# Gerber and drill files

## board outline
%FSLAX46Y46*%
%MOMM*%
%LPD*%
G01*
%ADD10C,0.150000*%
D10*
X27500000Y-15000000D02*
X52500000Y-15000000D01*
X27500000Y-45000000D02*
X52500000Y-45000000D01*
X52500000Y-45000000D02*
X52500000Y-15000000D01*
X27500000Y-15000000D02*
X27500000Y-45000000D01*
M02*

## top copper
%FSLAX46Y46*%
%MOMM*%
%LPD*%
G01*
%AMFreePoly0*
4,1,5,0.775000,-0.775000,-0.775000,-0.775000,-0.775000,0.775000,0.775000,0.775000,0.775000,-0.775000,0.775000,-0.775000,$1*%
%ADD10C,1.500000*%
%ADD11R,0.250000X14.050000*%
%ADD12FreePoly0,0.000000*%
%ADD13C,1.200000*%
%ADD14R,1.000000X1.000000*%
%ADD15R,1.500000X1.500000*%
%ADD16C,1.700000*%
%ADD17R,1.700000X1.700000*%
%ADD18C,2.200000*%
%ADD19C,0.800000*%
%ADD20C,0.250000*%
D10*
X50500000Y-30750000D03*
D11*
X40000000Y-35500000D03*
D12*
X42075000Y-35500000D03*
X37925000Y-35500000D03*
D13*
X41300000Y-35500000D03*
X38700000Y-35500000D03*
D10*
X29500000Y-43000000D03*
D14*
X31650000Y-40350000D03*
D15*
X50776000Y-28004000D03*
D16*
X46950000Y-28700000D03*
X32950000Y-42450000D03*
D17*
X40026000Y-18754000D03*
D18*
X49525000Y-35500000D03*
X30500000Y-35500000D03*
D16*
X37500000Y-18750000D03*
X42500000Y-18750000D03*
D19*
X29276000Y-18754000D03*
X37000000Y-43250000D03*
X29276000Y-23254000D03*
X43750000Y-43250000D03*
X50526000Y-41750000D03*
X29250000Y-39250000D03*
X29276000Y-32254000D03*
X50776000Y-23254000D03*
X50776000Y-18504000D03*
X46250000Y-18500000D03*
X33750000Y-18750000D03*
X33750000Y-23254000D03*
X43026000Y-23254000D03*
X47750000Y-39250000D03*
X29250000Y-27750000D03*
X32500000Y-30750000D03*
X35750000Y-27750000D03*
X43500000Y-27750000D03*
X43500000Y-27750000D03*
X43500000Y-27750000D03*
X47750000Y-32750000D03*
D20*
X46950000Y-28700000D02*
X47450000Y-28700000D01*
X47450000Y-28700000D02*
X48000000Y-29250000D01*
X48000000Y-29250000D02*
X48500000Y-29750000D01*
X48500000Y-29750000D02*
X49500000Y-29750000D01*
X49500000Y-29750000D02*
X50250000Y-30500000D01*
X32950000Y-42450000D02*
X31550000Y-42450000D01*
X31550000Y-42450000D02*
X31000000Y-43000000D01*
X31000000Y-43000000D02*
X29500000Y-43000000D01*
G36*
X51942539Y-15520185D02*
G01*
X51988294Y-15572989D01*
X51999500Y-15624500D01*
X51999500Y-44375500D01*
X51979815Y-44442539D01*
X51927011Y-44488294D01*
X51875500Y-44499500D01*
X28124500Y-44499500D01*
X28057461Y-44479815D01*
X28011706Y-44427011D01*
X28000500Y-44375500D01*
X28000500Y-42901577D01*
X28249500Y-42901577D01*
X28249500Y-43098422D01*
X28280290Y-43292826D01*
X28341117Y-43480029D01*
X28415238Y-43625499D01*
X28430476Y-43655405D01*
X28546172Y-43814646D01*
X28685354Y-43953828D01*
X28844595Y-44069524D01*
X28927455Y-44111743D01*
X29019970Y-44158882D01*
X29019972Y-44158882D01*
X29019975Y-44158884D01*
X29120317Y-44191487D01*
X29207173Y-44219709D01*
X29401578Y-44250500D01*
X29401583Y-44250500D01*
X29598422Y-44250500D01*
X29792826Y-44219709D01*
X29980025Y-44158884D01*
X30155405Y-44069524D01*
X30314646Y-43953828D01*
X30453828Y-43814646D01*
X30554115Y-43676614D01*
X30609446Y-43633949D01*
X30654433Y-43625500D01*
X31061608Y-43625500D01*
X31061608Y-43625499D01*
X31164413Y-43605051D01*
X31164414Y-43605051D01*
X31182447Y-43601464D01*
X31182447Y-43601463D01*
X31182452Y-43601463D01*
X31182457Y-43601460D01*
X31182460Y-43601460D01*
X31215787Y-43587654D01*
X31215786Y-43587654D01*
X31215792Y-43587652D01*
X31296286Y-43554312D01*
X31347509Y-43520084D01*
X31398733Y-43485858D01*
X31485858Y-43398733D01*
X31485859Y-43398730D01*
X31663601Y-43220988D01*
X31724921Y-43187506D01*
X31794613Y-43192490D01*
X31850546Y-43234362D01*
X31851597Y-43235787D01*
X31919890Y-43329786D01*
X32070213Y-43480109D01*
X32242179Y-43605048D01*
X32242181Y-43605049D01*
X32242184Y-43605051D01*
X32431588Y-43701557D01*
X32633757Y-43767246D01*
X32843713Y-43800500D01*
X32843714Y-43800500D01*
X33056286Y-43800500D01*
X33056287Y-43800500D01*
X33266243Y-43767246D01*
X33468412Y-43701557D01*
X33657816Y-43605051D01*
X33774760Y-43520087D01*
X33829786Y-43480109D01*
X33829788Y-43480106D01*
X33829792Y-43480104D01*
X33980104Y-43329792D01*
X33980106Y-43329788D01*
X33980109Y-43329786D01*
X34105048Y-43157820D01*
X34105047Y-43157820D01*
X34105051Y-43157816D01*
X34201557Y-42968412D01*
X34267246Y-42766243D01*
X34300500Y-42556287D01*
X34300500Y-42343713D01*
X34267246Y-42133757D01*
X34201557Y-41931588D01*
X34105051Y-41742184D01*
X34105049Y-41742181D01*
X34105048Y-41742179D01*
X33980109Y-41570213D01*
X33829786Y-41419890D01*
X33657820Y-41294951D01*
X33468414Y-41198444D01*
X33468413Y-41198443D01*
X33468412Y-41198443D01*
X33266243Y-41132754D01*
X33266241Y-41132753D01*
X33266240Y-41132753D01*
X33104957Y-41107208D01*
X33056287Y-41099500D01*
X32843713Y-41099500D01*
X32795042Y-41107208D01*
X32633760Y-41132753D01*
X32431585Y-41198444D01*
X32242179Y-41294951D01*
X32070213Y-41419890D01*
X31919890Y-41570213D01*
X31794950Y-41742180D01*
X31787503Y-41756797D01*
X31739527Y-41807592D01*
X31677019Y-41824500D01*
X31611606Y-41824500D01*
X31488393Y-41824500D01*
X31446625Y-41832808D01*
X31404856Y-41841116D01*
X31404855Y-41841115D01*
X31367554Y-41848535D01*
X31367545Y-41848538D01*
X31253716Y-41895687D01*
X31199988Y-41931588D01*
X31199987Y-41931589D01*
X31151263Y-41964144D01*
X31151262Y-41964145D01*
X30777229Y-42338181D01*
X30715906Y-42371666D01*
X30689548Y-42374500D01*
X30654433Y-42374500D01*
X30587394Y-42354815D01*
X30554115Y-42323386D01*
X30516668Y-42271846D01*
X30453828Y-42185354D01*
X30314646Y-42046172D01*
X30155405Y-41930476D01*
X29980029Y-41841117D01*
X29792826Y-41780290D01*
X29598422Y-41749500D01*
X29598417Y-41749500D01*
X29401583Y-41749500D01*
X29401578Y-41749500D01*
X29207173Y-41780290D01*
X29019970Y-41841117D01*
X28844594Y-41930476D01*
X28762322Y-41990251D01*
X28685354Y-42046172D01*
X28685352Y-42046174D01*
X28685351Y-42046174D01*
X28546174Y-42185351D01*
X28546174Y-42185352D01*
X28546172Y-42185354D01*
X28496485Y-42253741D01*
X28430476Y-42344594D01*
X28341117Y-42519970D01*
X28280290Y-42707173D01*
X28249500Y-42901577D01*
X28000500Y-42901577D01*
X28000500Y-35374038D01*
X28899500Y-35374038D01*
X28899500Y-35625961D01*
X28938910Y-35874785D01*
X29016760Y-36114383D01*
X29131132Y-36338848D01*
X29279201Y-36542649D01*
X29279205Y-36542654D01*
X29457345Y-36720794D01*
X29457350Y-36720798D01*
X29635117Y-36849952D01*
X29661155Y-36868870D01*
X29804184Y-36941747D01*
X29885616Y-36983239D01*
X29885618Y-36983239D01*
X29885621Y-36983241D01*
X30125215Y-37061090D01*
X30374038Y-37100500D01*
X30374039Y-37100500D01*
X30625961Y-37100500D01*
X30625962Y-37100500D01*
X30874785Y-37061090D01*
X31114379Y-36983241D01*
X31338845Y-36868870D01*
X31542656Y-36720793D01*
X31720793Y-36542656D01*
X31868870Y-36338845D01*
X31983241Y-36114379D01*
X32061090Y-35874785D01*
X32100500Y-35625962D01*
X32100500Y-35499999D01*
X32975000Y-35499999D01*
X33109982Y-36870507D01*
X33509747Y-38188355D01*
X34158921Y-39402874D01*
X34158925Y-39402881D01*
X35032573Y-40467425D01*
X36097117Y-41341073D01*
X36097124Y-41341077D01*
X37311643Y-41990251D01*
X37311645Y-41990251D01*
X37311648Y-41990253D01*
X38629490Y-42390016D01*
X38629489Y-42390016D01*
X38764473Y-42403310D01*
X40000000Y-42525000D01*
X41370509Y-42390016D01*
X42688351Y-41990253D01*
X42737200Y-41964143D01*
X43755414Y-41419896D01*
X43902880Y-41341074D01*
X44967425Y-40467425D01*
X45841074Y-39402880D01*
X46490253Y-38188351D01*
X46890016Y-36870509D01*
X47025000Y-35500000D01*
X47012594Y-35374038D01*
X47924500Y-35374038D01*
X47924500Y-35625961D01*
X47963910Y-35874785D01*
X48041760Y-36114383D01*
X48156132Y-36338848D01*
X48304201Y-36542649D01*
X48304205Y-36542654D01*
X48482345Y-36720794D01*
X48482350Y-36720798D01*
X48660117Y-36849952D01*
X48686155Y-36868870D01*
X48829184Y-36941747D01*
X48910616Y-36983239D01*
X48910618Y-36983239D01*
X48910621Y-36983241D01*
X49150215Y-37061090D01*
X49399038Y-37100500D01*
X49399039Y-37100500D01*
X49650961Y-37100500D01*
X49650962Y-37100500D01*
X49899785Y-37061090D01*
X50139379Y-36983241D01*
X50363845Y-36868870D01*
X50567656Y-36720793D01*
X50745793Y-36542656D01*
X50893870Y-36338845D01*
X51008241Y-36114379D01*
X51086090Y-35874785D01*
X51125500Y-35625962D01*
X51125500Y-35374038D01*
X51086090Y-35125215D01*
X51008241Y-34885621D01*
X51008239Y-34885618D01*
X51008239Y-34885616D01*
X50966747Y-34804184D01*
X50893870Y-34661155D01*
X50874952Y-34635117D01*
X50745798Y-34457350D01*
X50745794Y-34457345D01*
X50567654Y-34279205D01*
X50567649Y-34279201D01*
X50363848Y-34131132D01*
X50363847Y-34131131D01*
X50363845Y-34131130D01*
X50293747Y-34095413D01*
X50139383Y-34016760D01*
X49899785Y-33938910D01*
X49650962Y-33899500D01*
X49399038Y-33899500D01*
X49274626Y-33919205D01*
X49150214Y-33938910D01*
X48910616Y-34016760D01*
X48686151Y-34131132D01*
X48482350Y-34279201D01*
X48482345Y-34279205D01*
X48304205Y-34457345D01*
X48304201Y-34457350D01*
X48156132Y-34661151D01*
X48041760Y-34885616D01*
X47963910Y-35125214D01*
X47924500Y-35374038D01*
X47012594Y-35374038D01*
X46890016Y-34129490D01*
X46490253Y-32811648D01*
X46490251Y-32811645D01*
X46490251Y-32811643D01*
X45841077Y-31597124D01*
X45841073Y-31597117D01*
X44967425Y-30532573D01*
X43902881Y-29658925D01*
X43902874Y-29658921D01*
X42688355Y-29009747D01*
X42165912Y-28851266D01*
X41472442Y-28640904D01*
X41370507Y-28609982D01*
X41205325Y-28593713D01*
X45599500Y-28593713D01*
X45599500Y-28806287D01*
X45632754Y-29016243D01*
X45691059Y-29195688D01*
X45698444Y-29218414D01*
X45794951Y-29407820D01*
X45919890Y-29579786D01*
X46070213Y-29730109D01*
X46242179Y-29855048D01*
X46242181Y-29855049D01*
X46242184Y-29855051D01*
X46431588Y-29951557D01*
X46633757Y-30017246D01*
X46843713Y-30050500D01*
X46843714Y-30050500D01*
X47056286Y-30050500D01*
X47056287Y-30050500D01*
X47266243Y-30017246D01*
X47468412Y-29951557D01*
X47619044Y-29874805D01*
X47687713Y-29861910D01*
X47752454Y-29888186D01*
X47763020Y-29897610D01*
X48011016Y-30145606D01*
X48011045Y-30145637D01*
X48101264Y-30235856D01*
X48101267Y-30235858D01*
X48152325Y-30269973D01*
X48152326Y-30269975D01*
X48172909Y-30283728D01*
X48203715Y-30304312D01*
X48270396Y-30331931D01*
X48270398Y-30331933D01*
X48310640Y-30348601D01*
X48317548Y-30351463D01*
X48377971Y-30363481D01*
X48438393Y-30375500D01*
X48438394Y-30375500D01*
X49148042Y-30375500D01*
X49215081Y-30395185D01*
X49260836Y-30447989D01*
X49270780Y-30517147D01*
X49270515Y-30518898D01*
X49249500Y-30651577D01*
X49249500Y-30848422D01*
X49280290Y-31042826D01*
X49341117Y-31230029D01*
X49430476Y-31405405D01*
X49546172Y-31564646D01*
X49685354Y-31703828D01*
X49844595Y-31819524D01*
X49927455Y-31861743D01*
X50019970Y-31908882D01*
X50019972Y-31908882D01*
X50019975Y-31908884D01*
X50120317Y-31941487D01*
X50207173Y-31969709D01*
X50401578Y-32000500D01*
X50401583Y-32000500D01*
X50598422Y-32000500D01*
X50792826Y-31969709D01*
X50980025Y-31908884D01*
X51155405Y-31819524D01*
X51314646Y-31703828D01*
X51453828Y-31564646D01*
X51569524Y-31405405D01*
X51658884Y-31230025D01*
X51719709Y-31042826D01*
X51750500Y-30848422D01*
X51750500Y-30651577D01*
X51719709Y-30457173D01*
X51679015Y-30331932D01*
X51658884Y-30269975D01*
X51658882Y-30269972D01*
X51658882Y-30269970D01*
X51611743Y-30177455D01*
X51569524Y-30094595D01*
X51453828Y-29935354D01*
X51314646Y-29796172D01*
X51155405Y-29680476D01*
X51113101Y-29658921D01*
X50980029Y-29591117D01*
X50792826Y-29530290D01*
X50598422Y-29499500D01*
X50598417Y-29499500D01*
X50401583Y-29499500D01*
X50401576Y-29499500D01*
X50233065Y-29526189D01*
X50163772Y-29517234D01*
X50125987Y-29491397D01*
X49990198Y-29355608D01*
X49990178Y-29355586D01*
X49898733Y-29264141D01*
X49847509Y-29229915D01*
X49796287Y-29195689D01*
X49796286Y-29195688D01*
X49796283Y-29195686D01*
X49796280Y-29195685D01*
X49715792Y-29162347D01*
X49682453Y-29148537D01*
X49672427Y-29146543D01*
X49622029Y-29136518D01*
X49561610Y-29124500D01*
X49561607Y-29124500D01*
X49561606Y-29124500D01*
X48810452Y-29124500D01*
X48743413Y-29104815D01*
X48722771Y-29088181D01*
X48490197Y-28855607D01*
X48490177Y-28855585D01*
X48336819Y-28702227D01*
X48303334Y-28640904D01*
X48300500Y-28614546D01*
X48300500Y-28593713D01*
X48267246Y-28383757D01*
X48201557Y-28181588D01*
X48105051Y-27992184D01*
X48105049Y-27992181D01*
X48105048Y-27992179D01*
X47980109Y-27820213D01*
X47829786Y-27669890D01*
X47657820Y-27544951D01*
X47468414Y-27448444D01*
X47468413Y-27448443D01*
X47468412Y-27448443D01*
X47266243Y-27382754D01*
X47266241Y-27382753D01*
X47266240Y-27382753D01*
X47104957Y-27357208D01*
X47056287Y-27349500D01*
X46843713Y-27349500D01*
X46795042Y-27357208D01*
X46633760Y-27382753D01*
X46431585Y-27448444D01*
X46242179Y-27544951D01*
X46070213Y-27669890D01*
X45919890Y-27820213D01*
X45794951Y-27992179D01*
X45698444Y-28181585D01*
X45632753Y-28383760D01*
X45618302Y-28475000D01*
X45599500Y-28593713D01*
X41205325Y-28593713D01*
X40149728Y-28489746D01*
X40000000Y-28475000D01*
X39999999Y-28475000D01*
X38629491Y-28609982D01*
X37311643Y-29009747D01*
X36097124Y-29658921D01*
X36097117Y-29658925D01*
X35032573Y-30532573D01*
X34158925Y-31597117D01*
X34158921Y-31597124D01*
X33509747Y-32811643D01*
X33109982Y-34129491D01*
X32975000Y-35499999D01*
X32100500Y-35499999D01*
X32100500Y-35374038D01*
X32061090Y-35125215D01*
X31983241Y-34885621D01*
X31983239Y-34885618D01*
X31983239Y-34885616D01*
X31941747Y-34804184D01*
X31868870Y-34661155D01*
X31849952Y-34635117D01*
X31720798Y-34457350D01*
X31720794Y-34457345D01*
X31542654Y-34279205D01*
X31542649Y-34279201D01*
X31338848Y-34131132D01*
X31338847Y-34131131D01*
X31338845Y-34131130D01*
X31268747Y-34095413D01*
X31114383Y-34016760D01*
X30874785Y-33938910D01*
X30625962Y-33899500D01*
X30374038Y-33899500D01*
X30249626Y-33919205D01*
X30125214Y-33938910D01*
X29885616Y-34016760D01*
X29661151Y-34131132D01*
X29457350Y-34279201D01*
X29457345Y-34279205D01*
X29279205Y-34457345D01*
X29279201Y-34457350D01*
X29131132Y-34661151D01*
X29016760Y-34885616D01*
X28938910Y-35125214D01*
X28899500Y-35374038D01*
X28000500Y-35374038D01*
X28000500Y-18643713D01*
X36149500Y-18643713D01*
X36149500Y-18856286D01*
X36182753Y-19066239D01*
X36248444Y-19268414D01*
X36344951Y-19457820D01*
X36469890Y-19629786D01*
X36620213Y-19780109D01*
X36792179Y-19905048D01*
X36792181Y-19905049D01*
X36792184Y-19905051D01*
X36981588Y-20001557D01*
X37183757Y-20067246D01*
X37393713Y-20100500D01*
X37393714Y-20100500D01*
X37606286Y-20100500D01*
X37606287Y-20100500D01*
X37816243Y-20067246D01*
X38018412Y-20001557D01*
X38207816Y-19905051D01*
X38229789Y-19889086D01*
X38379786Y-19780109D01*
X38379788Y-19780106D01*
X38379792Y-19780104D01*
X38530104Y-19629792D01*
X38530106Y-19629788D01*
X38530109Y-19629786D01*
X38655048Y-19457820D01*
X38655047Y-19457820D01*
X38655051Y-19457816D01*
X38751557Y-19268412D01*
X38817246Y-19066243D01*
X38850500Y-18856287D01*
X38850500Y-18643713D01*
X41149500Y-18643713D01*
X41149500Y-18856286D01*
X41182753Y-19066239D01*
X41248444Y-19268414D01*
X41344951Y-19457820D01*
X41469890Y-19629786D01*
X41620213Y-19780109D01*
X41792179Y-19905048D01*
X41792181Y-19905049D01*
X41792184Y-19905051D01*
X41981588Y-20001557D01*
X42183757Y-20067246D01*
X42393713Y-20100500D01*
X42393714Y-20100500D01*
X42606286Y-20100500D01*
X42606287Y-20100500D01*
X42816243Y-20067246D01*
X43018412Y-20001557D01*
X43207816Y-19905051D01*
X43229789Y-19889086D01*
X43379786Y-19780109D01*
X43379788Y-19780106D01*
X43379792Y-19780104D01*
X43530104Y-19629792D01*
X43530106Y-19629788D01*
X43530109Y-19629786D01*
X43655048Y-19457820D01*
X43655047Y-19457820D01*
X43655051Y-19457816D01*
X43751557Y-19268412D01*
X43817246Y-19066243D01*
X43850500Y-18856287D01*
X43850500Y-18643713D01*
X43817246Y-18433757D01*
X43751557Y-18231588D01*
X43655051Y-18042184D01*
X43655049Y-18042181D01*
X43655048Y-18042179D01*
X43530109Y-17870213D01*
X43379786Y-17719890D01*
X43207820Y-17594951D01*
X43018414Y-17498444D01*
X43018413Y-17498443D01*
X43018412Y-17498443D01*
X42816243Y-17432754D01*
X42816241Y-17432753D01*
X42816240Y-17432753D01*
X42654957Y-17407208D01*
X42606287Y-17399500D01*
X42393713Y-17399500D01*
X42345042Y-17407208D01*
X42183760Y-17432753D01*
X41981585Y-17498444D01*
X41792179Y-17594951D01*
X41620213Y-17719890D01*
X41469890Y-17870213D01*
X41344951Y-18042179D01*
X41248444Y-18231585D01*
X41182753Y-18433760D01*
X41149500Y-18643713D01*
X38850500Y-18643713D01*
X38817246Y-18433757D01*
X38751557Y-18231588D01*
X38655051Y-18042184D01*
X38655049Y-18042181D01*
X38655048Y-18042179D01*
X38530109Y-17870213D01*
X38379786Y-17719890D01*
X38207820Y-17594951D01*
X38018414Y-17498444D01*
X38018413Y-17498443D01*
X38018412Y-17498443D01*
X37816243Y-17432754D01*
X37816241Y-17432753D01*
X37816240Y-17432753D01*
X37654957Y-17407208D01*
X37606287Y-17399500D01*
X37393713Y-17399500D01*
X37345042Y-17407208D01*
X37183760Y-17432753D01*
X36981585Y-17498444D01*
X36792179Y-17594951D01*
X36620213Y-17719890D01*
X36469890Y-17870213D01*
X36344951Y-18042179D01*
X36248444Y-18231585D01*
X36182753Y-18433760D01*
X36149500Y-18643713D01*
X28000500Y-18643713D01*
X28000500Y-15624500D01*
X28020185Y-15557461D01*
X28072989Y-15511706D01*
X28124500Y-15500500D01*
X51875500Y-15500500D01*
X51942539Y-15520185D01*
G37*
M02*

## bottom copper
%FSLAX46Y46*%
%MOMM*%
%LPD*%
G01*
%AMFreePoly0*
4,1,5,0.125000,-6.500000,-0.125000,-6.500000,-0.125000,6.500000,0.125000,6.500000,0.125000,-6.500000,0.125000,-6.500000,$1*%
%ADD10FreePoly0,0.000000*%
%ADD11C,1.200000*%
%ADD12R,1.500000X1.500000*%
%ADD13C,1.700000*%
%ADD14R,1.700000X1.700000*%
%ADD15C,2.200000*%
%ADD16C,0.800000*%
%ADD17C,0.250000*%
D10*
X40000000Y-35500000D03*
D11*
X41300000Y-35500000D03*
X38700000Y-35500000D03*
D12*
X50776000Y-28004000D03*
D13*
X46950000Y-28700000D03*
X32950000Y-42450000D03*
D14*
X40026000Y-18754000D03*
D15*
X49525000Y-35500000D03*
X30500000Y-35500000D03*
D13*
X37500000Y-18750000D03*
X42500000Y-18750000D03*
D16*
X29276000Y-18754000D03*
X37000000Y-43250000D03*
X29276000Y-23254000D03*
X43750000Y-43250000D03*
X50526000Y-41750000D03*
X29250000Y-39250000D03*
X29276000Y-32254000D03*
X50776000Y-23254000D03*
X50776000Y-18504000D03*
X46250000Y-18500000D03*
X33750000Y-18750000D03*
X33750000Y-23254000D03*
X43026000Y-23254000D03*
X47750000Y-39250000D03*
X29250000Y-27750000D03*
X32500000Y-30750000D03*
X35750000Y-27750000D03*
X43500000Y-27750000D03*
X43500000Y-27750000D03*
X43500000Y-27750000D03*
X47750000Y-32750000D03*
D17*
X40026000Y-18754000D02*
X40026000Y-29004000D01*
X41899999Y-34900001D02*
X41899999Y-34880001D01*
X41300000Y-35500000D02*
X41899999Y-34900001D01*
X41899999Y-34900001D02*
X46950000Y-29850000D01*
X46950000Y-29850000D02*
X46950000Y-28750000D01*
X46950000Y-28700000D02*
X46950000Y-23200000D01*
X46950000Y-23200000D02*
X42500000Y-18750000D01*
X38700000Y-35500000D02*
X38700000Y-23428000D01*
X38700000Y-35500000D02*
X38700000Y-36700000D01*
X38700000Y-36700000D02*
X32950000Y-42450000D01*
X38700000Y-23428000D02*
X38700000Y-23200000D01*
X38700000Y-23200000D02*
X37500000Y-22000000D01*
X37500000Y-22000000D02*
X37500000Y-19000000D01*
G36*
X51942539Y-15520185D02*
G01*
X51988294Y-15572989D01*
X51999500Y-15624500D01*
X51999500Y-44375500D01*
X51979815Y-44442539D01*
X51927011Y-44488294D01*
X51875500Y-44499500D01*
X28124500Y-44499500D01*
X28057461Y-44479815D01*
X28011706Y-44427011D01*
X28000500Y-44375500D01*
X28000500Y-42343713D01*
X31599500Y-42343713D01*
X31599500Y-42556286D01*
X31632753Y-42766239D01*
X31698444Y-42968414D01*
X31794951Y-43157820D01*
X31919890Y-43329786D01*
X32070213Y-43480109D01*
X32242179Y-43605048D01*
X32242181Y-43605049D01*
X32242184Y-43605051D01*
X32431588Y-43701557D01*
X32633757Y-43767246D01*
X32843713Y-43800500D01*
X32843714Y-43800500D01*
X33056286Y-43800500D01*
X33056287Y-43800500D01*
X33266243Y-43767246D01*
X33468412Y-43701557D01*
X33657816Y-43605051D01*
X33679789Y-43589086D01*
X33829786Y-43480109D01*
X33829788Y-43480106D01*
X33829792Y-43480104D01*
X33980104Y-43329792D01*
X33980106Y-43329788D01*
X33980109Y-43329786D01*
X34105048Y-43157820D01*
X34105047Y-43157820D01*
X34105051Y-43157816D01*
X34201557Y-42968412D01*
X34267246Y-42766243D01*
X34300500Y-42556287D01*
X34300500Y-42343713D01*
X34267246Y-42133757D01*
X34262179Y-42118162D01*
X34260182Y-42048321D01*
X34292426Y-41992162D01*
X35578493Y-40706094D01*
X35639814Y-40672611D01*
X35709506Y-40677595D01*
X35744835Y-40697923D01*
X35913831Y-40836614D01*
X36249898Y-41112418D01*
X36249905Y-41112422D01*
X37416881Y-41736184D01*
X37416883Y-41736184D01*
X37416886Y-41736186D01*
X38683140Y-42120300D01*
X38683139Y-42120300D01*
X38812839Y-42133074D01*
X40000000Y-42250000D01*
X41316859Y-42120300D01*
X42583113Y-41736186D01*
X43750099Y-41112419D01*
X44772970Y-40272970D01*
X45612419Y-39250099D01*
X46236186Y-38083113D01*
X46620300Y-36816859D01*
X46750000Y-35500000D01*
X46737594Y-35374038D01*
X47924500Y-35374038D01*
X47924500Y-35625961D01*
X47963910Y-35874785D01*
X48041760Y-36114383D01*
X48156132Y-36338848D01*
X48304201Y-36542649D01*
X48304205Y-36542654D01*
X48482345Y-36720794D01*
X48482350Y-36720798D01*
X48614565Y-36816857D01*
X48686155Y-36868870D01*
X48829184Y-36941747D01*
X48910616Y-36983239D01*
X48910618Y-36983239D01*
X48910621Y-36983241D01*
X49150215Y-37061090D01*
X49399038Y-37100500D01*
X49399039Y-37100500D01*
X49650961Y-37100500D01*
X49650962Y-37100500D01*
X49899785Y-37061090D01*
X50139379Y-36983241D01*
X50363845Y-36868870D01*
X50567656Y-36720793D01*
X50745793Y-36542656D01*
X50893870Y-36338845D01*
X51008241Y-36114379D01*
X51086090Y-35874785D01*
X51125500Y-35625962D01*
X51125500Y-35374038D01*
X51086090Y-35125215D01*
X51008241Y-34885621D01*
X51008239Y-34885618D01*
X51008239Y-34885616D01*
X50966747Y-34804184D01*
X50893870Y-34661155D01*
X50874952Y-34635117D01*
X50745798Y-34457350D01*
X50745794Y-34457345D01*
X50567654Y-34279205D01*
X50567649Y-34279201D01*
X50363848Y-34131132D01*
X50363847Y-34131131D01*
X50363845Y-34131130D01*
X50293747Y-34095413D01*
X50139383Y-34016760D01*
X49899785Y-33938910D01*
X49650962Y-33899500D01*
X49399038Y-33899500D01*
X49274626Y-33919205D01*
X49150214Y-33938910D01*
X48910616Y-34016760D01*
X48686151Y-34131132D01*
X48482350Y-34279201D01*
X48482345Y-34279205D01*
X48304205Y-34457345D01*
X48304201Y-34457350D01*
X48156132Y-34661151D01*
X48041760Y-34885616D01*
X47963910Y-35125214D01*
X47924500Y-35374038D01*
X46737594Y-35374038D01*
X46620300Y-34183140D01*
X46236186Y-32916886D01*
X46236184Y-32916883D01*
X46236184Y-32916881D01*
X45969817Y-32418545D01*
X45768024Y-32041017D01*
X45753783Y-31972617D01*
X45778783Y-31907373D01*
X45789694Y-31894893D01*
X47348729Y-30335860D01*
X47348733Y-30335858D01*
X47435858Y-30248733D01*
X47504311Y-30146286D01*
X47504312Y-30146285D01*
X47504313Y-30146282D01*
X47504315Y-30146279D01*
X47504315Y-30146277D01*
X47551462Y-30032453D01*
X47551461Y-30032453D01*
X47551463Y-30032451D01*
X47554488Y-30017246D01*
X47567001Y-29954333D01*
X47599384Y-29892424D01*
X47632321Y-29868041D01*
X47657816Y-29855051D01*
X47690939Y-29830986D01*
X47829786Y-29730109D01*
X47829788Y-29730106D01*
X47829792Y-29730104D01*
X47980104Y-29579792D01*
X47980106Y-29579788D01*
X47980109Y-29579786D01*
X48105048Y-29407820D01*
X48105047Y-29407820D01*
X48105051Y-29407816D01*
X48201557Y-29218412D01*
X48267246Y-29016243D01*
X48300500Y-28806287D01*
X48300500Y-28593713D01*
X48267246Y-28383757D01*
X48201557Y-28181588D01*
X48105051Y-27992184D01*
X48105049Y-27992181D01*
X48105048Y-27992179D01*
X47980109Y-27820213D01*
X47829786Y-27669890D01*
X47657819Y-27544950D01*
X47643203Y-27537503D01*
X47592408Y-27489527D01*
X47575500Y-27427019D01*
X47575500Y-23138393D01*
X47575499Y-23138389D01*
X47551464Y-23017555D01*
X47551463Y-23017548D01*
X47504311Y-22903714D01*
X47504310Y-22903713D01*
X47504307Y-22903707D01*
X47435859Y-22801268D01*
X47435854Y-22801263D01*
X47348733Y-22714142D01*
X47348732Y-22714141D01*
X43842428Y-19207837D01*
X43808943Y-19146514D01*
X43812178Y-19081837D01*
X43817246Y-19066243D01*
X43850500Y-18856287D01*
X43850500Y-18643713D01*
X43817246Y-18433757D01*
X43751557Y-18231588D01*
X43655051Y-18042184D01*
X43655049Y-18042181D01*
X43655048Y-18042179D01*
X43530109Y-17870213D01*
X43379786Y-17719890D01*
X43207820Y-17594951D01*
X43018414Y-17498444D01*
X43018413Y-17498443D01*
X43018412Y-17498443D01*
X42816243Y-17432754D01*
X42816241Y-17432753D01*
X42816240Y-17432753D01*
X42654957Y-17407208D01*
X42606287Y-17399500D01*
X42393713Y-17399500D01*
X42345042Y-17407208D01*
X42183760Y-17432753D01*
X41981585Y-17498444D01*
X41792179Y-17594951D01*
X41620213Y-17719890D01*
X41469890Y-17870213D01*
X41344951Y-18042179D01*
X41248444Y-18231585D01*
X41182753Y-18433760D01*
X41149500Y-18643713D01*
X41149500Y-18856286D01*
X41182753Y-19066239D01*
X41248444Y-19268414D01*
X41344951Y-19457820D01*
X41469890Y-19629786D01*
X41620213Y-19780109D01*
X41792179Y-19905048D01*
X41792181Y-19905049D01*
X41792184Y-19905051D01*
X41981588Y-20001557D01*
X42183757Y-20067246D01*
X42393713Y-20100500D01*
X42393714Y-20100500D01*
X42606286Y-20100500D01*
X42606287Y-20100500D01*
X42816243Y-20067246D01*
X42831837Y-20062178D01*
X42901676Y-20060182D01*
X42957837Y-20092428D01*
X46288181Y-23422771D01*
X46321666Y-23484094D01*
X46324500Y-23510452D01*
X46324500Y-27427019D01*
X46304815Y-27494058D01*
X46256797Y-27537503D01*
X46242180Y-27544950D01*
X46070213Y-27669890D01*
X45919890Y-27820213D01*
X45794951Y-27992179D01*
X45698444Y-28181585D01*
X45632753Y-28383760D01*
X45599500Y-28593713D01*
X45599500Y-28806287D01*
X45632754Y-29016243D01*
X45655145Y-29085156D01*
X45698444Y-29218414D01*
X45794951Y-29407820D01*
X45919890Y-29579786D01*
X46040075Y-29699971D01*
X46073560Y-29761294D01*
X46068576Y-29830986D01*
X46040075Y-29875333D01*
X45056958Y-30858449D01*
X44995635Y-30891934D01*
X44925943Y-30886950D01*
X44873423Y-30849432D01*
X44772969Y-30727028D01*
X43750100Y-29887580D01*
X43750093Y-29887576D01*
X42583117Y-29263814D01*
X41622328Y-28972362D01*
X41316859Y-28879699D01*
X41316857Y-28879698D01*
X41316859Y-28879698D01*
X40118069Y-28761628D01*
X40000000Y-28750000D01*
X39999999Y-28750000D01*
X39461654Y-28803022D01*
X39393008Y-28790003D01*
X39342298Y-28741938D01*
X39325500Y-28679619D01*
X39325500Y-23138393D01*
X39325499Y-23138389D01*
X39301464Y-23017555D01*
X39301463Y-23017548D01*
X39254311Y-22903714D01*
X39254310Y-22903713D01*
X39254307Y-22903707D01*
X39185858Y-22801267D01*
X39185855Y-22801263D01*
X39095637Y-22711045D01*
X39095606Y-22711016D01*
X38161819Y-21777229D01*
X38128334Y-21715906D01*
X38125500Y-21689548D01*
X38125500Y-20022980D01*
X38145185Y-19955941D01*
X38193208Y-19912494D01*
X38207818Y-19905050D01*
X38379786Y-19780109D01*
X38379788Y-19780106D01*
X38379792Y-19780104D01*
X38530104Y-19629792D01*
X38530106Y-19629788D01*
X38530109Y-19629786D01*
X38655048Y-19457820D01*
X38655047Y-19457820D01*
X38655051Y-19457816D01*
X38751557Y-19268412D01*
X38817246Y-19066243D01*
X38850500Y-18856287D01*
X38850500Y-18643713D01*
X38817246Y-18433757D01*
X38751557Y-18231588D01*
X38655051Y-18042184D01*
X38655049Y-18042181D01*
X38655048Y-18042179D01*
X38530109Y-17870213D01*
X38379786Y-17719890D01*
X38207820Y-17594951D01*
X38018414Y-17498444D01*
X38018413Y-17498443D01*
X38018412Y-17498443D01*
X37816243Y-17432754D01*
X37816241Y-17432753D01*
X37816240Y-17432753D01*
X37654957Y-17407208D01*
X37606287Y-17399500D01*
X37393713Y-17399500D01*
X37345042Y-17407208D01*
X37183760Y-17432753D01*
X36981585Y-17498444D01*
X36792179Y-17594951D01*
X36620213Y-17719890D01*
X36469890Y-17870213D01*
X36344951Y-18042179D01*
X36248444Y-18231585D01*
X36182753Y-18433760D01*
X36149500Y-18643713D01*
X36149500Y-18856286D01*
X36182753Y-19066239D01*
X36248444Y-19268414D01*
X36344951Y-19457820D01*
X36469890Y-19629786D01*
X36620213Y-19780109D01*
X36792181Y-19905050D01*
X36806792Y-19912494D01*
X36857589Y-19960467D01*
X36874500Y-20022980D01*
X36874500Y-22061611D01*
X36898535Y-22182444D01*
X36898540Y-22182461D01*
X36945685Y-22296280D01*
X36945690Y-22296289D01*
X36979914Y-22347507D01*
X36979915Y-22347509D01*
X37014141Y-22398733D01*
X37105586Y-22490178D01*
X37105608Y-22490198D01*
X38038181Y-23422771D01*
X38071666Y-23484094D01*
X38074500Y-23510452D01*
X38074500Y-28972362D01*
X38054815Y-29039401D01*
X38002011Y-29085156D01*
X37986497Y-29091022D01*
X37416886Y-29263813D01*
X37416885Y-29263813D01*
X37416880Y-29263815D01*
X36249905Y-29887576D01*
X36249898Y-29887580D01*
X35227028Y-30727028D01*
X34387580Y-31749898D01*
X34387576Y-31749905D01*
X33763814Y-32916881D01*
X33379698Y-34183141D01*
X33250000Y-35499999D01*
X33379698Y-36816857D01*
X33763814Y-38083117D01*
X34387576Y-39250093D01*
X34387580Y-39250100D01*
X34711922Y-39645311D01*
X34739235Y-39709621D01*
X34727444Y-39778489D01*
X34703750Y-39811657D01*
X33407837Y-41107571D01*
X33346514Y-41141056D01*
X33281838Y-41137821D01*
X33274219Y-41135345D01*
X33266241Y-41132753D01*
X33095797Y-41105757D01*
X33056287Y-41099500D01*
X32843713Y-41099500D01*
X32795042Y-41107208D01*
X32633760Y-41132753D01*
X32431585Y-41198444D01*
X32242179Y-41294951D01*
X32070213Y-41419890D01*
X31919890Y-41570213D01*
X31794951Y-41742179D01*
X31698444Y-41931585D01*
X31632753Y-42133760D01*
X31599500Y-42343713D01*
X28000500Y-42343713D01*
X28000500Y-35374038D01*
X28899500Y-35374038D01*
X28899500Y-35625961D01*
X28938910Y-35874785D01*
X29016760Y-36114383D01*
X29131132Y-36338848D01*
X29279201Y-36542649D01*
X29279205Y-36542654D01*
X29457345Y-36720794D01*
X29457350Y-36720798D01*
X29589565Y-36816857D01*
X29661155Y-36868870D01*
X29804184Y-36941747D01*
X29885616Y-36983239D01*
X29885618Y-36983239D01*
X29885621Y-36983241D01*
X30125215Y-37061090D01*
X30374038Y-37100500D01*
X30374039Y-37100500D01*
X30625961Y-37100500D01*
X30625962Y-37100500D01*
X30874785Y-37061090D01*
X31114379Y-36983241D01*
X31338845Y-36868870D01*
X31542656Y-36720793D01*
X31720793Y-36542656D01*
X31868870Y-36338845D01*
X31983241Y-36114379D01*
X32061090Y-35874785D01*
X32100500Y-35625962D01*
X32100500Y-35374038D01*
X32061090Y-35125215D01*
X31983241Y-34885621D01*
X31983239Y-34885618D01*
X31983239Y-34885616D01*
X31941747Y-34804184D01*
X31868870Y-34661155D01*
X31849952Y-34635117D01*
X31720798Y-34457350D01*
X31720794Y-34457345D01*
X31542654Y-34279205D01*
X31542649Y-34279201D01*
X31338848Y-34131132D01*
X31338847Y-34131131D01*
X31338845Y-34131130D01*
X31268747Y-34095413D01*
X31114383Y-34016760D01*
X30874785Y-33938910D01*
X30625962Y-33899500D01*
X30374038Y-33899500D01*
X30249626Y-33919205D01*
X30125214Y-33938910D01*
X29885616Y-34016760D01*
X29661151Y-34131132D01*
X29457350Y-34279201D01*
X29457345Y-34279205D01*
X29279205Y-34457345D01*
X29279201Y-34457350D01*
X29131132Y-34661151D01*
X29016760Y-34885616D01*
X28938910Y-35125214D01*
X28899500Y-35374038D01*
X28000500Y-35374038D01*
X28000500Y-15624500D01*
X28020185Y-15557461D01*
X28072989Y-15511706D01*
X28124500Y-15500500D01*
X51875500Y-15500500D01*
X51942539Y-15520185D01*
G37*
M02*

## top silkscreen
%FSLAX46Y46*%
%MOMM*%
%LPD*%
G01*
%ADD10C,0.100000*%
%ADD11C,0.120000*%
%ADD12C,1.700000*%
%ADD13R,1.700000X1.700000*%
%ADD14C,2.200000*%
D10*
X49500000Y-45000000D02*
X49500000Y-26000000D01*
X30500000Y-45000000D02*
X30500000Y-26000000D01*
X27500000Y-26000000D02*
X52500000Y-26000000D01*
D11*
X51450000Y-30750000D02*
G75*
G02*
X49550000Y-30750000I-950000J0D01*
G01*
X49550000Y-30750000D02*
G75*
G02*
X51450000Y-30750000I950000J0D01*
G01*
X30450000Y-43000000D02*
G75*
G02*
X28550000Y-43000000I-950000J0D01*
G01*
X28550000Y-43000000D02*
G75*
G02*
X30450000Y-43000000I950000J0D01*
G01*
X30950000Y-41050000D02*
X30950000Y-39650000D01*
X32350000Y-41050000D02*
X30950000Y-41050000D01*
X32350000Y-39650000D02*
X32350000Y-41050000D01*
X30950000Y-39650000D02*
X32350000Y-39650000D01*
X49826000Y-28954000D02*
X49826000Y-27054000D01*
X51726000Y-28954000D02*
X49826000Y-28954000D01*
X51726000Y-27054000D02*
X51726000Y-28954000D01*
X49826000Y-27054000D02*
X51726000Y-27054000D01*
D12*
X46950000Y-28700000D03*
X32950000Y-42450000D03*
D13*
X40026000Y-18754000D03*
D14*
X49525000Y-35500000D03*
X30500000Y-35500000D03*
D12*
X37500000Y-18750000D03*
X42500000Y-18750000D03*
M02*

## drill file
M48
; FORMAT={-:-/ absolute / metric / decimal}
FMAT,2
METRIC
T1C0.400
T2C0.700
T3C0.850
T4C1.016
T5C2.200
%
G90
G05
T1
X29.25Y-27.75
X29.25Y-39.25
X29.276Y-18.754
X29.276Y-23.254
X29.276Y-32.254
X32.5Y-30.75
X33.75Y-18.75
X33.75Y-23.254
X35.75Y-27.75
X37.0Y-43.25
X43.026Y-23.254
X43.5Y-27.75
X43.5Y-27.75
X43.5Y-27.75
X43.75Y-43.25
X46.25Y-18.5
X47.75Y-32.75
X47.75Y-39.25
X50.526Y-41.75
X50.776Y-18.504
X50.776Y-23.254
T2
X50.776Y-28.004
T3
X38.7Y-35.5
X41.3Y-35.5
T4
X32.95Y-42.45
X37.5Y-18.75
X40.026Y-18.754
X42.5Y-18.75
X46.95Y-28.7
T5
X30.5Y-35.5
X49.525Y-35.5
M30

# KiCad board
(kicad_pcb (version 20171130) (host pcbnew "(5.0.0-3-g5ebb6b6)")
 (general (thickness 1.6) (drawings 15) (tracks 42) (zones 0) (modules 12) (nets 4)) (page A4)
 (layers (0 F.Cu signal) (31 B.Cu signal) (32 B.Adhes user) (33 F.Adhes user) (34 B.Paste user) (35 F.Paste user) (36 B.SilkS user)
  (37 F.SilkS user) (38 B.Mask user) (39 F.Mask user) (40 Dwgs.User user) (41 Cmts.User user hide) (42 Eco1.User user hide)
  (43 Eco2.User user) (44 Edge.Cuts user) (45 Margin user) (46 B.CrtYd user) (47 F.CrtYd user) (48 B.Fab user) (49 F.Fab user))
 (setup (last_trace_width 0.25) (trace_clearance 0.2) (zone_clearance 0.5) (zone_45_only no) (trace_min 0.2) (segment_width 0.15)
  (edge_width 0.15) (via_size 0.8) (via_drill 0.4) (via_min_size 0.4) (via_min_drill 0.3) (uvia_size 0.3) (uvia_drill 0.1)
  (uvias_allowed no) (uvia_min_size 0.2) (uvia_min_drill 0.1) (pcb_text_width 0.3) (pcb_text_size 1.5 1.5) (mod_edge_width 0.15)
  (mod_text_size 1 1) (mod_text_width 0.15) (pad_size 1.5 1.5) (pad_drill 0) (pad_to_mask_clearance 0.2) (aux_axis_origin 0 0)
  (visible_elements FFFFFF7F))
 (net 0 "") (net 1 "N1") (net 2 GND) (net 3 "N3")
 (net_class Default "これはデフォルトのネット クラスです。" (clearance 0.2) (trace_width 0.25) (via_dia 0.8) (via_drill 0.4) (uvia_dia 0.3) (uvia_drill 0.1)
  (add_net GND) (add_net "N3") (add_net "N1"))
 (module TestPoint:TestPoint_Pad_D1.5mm (layer F.Cu) (at 50.5 30.75)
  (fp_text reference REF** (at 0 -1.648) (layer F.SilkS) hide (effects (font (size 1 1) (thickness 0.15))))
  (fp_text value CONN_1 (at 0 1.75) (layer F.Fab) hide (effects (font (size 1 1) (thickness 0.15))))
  (fp_circle (center 0 0) (end 0 0.95) (layer F.SilkS) (width 0.12))
  (pad 12 smd circle (at 0 0) (size 1.5 1.5) (layers F.Cu F.Mask) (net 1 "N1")))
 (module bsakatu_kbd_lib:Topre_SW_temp (layer F.Cu) (at 40 35.5) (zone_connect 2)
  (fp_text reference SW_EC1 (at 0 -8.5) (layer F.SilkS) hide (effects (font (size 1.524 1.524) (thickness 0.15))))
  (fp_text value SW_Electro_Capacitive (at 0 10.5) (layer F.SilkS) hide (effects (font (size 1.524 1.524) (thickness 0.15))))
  (pad 3 smd rect (at 0 0) (size 0.25 14.05) (layers F.Cu) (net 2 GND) (zone_connect 2))
  (pad 2 smd custom (at 2.075 0) (size 1.55 1.55) (layers F.Cu) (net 1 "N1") (zone_connect 0) (options (clearance outline) (anchor rect))
   (primitives))
  (pad 1 smd custom (at -2.075 0) (size 1.55 1.55) (layers F.Cu) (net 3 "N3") (zone_connect 0) (options (clearance outline) (anchor rect))
   (primitives))
  (pad "" smd custom (at 0 0) (size 0.25 13) (layers B.Cu) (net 2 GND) (zone_connect 2) (options (clearance outline) (anchor rect))
   (primitives))
  (pad 2 thru_hole circle (at 1.3 0) (size 1.2 1.2) (drill 0.85) (layers *.Cu *.Mask) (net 1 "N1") (zone_connect 2))
  (pad 1 thru_hole circle (at -1.3 0) (size 1.2 1.2) (drill 0.85) (layers *.Cu *.Mask) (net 3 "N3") (zone_connect 2)))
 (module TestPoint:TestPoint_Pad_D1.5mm (layer F.Cu) (at 29.5 43)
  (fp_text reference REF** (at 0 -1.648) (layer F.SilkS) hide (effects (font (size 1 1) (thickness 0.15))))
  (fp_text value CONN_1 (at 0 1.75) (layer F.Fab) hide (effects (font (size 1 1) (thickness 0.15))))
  (fp_circle (center 0 0) (end 0 0.95) (layer F.SilkS) (width 0.12))
  (pad 11 smd circle (at 0 0) (size 1.5 1.5) (layers F.Cu F.Mask) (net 3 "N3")))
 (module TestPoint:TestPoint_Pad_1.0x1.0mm (layer F.Cu) (at 31.65 40.35)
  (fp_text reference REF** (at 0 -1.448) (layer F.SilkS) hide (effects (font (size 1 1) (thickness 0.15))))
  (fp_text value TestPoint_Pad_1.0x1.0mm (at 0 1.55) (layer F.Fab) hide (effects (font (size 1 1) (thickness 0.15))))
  (fp_line (start -0.7 0.7) (end -0.7 -0.7) (layer F.SilkS) (width 0.12))
  (fp_line (start 0.7 0.7) (end -0.7 0.7) (layer F.SilkS) (width 0.12))
  (fp_line (start 0.7 -0.7) (end 0.7 0.7) (layer F.SilkS) (width 0.12))
  (fp_line (start -0.7 -0.7) (end 0.7 -0.7) (layer F.SilkS) (width 0.12))
  (pad 7 smd rect (at 0 0) (size 1 1) (layers F.Cu F.Mask) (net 2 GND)))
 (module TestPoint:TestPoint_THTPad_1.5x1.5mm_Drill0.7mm (layer F.Cu) (at 50.776 28.004)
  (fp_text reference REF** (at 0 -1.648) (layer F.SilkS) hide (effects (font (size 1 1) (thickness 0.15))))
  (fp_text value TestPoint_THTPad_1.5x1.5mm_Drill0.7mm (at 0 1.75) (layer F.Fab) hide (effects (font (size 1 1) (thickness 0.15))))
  (fp_line (start -0.95 0.95) (end -0.95 -0.95) (layer F.SilkS) (width 0.12))
  (fp_line (start 0.95 0.95) (end -0.95 0.95) (layer F.SilkS) (width 0.12))
  (fp_line (start 0.95 -0.95) (end 0.95 0.95) (layer F.SilkS) (width 0.12))
  (fp_line (start -0.95 -0.95) (end 0.95 -0.95) (layer F.SilkS) (width 0.12))
  (pad 8 thru_hole rect (at 0 0) (size 1.5 1.5) (drill 0.7) (layers *.Cu *.Mask) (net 2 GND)))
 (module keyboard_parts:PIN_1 (layer F.Cu) (at 46.95 28.7)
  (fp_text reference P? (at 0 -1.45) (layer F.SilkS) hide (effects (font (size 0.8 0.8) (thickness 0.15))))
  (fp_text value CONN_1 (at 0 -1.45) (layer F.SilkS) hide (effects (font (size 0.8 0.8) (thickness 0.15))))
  (pad 10 thru_hole circle (at 0 0) (size 1.7 1.7) (drill 1.016) (layers *.Cu *.Mask F.SilkS) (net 1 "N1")))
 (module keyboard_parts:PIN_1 (layer F.Cu) (at 32.95 42.45)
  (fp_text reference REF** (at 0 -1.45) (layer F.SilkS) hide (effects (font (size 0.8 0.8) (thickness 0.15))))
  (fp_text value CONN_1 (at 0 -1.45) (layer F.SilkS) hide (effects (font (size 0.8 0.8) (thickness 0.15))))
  (pad 9 thru_hole circle (at 0 0) (size 1.7 1.7) (drill 1.016) (layers *.Cu *.SilkS *.Mask) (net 3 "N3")))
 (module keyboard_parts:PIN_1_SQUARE (layer F.Cu) (at 40.026 18.754)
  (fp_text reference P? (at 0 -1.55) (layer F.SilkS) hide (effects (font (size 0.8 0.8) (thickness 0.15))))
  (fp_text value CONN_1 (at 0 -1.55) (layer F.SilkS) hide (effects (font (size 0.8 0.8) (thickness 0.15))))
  (pad 4 thru_hole rect (at 0 0) (size 1.7 1.7) (drill 1.016) (layers *.Cu *.Mask F.SilkS) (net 2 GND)))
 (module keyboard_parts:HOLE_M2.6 (layer F.Cu) (at 49.525 35.5)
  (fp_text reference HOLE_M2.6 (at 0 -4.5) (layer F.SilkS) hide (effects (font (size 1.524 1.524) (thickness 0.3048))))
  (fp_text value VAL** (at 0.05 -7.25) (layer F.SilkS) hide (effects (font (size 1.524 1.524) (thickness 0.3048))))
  (pad "" thru_hole circle (at 0 0) (size 2.2 2.2) (drill 2.2) (layers *.Cu *.SilkS *.Mask)))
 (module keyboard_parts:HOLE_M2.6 (layer F.Cu) (at 30.5 35.5)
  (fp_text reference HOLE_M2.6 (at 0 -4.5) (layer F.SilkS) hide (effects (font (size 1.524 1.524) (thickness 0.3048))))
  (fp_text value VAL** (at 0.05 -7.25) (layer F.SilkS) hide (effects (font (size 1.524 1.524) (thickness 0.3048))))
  (pad "" thru_hole circle (at 0 0) (size 2.2 2.2) (drill 2.2) (layers *.Cu *.SilkS *.Mask)))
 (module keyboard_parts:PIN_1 (layer F.Cu) (at 37.5 18.75)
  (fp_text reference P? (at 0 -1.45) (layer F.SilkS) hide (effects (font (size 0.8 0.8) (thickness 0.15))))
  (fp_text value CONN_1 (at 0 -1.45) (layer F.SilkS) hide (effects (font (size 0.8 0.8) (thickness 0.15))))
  (pad 5 thru_hole circle (at 0 0) (size 1.7 1.7) (drill 1.016) (layers *.Cu *.Mask F.SilkS) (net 3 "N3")))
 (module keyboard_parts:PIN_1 (layer F.Cu) (at 42.5 18.75)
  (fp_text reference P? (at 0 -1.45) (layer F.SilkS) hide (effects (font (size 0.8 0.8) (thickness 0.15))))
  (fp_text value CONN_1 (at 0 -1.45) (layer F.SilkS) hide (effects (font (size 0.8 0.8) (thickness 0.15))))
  (pad 6 thru_hole circle (at 0 0) (size 1.7 1.7) (drill 1.016) (layers *.Cu *.Mask F.SilkS) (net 1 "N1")))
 (gr_line (start 49.5 45) (end 49.5 26) (layer F.SilkS) (width 0.1))
 (gr_line (start 30.5 45) (end 30.5 26) (layer F.SilkS) (width 0.1))
 (gr_line (start 27.5 26) (end 52.5 26) (layer F.SilkS) (width 0.1))
 (gr_line (start 27.5 15) (end 52.5 15) (layer Edge.Cuts) (width 0.15))
 (gr_line (start 27.5 45) (end 52.5 45) (layer Edge.Cuts) (width 0.15))
 (gr_line (start 52.5 45) (end 52.5 15) (layer Edge.Cuts) (width 0.15))
 (gr_line (start 27.5 15) (end 27.5 45) (layer Edge.Cuts) (width 0.15))
 (via (at 29.276 18.754) (size 0.8) (drill 0.4) (layers F.Cu B.Cu) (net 2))
 (via (at 37 43.25) (size 0.8) (drill 0.4) (layers F.Cu B.Cu) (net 2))
 (via (at 29.276 23.254) (size 0.8) (drill 0.4) (layers F.Cu B.Cu) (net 2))
 (segment (start 40.026 18.754) (end 40.026 29.004) (width 0.25) (layer B.Cu) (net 2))
 (via (at 43.75 43.25) (size 0.8) (drill 0.4) (layers F.Cu B.Cu) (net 2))
 (via (at 50.526 41.75) (size 0.8) (drill 0.4) (layers F.Cu B.Cu) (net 2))
 (via (at 29.25 39.25) (size 0.8) (drill 0.4) (layers F.Cu B.Cu) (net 2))
 (via (at 29.276 32.254) (size 0.8) (drill 0.4) (layers F.Cu B.Cu) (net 2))
 (via (at 50.776 23.254) (size 0.8) (drill 0.4) (layers F.Cu B.Cu) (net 2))
 (via (at 50.776 18.504) (size 0.8) (drill 0.4) (layers F.Cu B.Cu) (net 2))
 (via (at 46.25 18.5) (size 0.8) (drill 0.4) (layers F.Cu B.Cu) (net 2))
 (via (at 33.75 18.75) (size 0.8) (drill 0.4) (layers F.Cu B.Cu) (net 2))
 (via (at 33.75 23.254) (size 0.8) (drill 0.4) (layers F.Cu B.Cu) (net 2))
 (via (at 43.026 23.254) (size 0.8) (drill 0.4) (layers F.Cu B.Cu) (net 2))
 (via (at 47.75 39.25) (size 0.8) (drill 0.4) (layers F.Cu B.Cu) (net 2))
 (via (at 29.25 27.75) (size 0.8) (drill 0.4) (layers F.Cu B.Cu) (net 2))
 (via (at 32.5 30.75) (size 0.8) (drill 0.4) (layers F.Cu B.Cu) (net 2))
 (via (at 35.75 27.75) (size 0.8) (drill 0.4) (layers F.Cu B.Cu) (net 2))
 (via (at 43.5 27.75) (size 0.8) (drill 0.4) (layers F.Cu B.Cu) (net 2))
 (via (at 43.5 27.75) (size 0.8) (drill 0.4) (layers F.Cu B.Cu) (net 2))
 (via (at 43.5 27.75) (size 0.8) (drill 0.4) (layers F.Cu B.Cu) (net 2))
 (via (at 47.75 32.75) (size 0.8) (drill 0.4) (layers F.Cu B.Cu) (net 2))
 (segment (start 41.899999 34.900001) (end 41.899999 34.880001) (width 0.25) (layer B.Cu) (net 1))
 (segment (start 41.3 35.5) (end 41.899999 34.900001) (width 0.25) (layer B.Cu) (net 1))
 (segment (start 41.899999 34.900001) (end 46.95 29.85) (width 0.25) (layer B.Cu) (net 1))
 (segment (start 46.95 29.85) (end 46.95 28.75) (width 0.25) (layer B.Cu) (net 1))
 (segment (start 46.95 28.7) (end 46.95 23.2) (width 0.25) (layer B.Cu) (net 1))
 (segment (start 46.95 23.2) (end 42.5 18.75) (width 0.25) (layer B.Cu) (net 1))
 (segment (start 46.95 28.7) (end 47.45 28.7) (width 0.25) (layer F.Cu) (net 1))
 (segment (start 47.45 28.7) (end 48 29.25) (width 0.25) (layer F.Cu) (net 1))
 (segment (start 48 29.25) (end 48.5 29.75) (width 0.25) (layer F.Cu) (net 1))
 (segment (start 48.5 29.75) (end 49.5 29.75) (width 0.25) (layer F.Cu) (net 1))
 (segment (start 49.5 29.75) (end 50.25 30.5) (width 0.25) (layer F.Cu) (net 1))
 (segment (start 38.7 35.5) (end 38.7 23.428) (width 0.25) (layer B.Cu) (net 3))
 (segment (start 38.7 35.5) (end 38.7 36.7) (width 0.25) (layer B.Cu) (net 3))
 (segment (start 38.7 36.7) (end 32.95 42.45) (width 0.25) (layer B.Cu) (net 3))
 (segment (start 32.95 42.45) (end 31.55 42.45) (width 0.25) (layer F.Cu) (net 3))
 (segment (start 31.55 42.45) (end 31 43) (width 0.25) (layer F.Cu) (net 3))
 (segment (start 31 43) (end 29.5 43) (width 0.25) (layer F.Cu) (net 3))
 (segment (start 38.7 23.428) (end 38.7 23.2) (width 0.25) (layer B.Cu) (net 3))
 (segment (start 38.7 23.2) (end 37.5 22) (width 0.25) (layer B.Cu) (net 3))
 (segment (start 37.5 22) (end 37.5 19) (width 0.25) (layer B.Cu) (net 3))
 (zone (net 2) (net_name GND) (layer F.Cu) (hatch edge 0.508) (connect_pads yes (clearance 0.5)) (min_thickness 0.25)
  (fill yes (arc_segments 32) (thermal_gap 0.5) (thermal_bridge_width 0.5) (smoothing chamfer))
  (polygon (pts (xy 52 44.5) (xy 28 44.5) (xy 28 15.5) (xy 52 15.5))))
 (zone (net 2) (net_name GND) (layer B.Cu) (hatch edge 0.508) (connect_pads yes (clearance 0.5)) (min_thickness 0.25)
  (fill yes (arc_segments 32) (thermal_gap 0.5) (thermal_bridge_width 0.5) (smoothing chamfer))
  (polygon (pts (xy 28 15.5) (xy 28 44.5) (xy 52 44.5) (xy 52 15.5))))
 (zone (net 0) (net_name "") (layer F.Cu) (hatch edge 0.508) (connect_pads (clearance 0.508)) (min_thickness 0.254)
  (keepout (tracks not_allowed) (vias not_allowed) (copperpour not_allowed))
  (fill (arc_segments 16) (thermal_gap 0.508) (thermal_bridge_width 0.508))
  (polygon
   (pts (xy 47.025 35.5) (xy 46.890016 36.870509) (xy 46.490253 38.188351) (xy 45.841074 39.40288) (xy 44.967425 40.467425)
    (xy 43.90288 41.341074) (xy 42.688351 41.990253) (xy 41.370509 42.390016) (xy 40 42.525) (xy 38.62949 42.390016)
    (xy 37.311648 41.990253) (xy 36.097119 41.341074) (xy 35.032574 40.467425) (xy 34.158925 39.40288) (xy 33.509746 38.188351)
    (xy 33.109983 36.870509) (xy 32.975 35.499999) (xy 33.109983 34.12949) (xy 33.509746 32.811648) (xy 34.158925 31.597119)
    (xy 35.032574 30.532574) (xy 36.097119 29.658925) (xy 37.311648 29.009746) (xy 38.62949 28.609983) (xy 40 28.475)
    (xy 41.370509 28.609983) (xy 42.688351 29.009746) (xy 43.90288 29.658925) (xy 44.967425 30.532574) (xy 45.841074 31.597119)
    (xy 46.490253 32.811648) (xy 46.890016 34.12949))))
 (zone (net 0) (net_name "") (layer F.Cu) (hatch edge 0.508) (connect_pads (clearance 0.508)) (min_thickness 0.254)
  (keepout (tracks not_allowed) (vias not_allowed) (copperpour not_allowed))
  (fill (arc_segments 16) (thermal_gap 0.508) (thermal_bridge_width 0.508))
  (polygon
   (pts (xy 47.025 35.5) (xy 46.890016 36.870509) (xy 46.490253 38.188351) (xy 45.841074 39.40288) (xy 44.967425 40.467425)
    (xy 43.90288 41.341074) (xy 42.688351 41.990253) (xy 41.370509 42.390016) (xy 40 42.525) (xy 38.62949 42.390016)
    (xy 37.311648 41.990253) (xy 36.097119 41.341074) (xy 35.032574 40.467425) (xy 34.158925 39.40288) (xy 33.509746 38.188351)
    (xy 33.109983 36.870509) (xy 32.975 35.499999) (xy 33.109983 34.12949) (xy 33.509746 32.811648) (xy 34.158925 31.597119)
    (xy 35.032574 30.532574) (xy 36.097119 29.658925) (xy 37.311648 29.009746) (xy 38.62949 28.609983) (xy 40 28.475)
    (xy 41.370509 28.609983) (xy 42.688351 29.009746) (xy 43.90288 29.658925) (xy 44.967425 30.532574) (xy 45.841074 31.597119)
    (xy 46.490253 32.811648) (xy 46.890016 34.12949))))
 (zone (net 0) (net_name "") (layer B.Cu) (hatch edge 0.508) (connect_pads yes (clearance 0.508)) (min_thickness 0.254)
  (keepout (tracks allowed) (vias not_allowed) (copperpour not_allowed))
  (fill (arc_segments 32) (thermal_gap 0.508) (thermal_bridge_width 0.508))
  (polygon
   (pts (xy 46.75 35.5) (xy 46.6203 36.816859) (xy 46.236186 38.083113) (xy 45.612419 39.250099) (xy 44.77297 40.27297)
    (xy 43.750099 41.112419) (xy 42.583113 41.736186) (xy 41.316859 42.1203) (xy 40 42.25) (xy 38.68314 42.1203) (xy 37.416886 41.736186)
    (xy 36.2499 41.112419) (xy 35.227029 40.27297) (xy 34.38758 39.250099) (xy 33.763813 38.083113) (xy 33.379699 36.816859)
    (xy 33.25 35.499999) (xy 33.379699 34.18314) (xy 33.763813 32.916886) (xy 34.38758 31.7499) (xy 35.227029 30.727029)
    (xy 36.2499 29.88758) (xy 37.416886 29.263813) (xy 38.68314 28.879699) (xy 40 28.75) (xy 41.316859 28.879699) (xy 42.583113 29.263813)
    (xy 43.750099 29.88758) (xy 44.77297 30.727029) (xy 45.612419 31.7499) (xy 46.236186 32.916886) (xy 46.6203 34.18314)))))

